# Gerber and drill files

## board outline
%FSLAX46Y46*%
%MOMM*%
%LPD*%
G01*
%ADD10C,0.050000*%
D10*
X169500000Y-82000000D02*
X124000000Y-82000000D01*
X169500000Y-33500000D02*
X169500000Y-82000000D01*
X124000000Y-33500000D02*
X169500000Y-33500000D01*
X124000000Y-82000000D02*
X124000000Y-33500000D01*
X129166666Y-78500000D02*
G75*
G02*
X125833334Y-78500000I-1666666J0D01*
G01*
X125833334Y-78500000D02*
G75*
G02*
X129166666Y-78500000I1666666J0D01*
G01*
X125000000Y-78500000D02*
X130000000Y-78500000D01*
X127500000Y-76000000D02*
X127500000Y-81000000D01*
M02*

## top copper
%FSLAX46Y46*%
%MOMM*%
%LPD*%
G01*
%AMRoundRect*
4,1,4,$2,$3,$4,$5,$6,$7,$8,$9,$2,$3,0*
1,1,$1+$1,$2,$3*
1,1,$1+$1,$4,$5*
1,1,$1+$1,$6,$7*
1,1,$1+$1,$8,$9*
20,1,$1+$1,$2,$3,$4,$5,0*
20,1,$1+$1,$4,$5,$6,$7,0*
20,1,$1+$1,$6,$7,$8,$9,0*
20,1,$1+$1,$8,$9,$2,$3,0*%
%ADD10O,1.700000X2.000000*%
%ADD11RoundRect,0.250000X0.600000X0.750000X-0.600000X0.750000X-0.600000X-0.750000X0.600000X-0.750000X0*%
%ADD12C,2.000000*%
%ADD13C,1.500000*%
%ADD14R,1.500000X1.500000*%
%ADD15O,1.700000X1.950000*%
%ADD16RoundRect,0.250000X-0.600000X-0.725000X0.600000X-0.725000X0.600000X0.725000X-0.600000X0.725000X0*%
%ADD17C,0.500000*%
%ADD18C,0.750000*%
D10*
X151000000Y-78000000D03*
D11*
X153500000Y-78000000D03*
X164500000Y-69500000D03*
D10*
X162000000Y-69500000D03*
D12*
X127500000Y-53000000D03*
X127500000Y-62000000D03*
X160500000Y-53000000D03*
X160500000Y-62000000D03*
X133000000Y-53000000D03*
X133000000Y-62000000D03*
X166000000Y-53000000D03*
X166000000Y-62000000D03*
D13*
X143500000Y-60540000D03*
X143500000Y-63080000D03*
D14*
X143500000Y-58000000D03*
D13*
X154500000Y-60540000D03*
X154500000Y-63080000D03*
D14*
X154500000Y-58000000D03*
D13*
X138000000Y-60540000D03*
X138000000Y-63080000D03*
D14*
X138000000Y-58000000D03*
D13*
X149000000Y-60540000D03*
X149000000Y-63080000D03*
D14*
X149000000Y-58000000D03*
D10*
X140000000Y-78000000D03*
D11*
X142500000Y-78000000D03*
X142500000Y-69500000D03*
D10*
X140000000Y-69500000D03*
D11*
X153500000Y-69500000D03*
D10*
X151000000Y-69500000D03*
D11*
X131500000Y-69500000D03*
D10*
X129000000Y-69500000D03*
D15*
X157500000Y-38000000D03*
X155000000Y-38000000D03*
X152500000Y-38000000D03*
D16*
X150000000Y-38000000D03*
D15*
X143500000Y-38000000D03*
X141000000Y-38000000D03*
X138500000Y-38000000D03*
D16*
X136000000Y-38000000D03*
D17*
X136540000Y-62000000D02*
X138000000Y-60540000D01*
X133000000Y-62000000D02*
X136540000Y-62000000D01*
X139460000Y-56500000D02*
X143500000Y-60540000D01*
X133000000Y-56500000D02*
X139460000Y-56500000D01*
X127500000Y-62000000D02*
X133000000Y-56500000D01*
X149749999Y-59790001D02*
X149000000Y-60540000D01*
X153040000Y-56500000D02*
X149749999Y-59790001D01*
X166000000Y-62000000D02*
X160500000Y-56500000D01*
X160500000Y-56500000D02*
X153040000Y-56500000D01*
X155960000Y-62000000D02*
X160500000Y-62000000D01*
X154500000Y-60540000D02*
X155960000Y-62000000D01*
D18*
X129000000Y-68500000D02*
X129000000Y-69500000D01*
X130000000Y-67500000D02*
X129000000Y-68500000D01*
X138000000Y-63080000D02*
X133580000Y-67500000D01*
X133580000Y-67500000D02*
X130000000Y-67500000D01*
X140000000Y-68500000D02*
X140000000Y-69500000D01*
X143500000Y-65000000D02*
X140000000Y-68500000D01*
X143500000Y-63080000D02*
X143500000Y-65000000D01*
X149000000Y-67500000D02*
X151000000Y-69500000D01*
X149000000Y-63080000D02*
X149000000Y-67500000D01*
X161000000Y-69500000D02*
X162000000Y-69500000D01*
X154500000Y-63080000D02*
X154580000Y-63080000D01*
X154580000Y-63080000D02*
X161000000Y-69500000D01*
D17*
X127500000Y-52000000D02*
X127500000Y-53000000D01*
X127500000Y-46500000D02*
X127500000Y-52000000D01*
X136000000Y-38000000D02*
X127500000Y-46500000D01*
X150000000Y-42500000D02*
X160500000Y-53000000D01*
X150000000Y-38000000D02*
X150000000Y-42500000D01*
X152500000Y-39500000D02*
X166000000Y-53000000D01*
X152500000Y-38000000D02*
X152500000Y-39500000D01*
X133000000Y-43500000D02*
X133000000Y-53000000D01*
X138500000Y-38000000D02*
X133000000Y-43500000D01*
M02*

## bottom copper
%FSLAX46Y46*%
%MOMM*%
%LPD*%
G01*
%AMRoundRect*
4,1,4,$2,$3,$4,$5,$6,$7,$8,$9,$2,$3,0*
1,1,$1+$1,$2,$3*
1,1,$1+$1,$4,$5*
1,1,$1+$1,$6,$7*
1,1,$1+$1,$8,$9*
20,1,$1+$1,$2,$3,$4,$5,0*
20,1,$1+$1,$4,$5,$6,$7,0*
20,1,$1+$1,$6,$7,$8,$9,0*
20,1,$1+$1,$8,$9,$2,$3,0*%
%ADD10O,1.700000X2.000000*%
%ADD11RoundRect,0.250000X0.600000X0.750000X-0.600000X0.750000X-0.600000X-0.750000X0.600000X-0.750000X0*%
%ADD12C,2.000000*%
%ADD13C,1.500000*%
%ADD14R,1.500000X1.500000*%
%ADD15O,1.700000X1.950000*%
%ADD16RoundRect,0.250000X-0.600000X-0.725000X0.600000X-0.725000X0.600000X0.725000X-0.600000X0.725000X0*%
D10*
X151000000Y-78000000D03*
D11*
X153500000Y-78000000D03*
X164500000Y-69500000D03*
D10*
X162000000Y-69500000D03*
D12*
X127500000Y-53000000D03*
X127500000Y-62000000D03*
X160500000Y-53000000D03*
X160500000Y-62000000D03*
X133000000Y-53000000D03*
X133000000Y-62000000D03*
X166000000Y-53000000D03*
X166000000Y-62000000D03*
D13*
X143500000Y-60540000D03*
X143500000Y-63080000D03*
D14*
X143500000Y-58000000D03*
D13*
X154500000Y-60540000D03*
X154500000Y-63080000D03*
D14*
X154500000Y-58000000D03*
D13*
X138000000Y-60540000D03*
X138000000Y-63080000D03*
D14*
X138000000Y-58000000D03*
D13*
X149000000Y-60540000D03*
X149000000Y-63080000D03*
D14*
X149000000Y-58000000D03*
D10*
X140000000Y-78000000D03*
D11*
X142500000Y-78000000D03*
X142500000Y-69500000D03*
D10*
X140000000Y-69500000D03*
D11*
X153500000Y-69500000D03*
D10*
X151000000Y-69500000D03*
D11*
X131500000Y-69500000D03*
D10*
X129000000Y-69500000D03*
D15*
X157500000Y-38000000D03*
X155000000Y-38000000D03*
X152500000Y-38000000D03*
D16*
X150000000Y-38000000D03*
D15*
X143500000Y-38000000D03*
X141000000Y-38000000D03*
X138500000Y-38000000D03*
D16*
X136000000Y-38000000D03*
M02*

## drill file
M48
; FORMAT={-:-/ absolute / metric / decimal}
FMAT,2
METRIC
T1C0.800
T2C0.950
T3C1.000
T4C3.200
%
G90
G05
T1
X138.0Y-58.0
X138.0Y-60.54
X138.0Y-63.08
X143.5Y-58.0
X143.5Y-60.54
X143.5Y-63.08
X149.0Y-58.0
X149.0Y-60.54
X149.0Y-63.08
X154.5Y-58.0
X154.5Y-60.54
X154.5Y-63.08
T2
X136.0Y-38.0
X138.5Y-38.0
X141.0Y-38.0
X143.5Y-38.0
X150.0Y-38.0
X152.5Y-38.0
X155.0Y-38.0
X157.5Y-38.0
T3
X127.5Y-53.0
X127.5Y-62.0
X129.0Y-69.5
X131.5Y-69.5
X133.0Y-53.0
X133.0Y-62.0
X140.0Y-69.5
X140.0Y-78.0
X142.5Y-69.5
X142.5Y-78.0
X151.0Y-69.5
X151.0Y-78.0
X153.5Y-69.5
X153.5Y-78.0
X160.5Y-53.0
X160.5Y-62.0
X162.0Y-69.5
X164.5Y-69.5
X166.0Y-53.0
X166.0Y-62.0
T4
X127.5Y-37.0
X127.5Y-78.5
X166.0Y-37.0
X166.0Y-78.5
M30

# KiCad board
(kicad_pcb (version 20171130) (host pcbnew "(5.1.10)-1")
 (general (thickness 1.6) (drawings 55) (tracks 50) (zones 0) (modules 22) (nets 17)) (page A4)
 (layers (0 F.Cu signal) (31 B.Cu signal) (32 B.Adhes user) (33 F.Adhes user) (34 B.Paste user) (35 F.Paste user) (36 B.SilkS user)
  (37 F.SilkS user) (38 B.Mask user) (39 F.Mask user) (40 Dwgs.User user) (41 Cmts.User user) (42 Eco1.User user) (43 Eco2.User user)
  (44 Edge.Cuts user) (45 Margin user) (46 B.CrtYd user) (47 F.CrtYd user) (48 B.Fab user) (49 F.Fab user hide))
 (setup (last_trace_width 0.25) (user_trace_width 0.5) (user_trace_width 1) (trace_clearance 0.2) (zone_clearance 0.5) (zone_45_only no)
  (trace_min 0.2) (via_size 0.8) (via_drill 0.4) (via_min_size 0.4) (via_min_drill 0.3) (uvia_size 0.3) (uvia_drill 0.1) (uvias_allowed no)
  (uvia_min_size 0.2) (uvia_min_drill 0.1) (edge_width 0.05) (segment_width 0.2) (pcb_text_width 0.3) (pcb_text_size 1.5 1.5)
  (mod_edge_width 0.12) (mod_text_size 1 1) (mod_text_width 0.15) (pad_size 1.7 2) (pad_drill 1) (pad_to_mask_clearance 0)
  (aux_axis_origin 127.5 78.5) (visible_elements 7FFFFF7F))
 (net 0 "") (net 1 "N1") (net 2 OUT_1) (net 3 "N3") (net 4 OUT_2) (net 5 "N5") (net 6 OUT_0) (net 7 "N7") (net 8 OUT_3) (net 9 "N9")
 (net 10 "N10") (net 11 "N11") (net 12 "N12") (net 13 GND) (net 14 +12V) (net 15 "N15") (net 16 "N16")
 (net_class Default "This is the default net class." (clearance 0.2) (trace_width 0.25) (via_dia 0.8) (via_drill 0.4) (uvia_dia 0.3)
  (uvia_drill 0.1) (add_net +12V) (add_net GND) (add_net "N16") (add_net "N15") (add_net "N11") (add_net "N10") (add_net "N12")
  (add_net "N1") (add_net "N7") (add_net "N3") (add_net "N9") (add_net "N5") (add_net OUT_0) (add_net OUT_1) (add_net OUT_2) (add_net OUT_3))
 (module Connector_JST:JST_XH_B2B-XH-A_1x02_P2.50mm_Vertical (layer F.Cu) (at 153.5 78 180)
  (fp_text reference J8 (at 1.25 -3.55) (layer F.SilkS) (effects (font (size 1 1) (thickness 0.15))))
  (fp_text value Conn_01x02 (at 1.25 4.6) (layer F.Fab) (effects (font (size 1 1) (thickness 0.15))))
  (pad 2 thru_hole oval (at 2.5 0 180) (size 1.7 2) (drill 1) (layers *.Cu *.Mask))
  (pad 1 thru_hole roundrect (at 0 0 180) (size 1.7 2) (drill 1) (layers *.Cu *.Mask) (roundrect_rratio 0.1470588235294118)))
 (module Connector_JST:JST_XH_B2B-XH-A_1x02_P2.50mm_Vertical (layer F.Cu) (at 164.5 69.5 180)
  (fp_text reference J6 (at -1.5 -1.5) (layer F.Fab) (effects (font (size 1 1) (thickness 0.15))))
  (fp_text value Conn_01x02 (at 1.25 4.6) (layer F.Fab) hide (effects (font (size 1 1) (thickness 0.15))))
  (pad 1 thru_hole roundrect (at 0 0 180) (size 1.7 2) (drill 1) (layers *.Cu *.Mask) (roundrect_rratio 0.1470588235294118))
  (pad 2 thru_hole oval (at 2.5 0 180) (size 1.7 2) (drill 1) (layers *.Cu *.Mask) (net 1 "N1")))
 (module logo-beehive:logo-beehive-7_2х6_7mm (layer F.Cu) (at 133 77 90)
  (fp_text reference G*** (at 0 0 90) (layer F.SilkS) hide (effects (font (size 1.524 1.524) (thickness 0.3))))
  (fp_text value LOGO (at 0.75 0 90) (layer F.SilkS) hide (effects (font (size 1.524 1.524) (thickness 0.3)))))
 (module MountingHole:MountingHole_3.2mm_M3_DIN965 (layer F.Cu) (at 166 37 270)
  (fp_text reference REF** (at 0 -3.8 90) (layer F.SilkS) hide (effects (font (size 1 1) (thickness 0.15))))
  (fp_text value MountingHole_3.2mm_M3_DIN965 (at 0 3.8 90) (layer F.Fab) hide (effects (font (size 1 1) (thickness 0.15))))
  (pad 1 np_thru_hole circle (at 0 0 270) (size 3.2 3.2) (drill 3.2) (layers *.Cu *.Mask)))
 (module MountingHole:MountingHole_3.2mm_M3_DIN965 (layer F.Cu) (at 166 78.5 180)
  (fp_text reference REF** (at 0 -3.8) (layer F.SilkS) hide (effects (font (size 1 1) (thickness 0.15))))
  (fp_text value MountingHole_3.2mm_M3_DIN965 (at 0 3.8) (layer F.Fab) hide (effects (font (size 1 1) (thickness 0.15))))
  (pad 1 np_thru_hole circle (at 0 0 180) (size 3.2 3.2) (drill 3.2) (layers *.Cu *.Mask)))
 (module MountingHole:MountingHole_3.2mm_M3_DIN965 (layer F.Cu) (at 127.5 78.5 90)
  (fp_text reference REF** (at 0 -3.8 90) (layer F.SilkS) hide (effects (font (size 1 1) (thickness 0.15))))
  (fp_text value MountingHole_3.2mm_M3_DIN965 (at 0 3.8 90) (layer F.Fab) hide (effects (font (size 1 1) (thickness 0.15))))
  (pad 1 np_thru_hole circle (at 0 0 90) (size 3.2 3.2) (drill 3.2) (layers *.Cu *.Mask)))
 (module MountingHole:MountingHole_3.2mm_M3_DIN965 (layer F.Cu) (at 127.5 37 90)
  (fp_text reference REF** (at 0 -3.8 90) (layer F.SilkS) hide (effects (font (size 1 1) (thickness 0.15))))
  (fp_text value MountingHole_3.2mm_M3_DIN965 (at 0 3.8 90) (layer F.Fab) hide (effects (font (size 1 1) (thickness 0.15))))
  (pad 1 np_thru_hole circle (at 0 0 90) (size 3.2 3.2) (drill 3.2) (layers *.Cu *.Mask)))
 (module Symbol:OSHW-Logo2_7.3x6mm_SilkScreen (layer F.Cu) (at 147 51)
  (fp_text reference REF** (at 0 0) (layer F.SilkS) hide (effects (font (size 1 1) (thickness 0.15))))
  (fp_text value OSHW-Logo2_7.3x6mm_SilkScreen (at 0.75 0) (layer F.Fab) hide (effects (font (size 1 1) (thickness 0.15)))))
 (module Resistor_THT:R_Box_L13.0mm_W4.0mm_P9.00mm (layer F.Cu) (at 127.5 53 270)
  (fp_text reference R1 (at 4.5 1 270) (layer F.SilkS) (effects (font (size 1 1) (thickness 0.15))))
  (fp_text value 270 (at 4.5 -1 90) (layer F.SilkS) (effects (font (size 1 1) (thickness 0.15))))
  (pad 1 thru_hole circle (at 0 0 270) (size 2 2) (drill 1) (layers *.Cu *.Mask) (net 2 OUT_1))
  (pad 2 thru_hole circle (at 9 0 270) (size 2 2) (drill 1) (layers *.Cu *.Mask) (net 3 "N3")))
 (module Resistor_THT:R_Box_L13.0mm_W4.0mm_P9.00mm (layer F.Cu) (at 160.5 53 270)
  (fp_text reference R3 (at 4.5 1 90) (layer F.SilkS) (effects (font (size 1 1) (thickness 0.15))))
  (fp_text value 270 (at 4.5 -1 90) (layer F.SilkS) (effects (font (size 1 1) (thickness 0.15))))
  (pad 1 thru_hole circle (at 0 0 270) (size 2 2) (drill 1) (layers *.Cu *.Mask) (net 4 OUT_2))
  (pad 2 thru_hole circle (at 9 0 270) (size 2 2) (drill 1) (layers *.Cu *.Mask) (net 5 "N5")))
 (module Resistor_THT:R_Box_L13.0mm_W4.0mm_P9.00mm (layer F.Cu) (at 133 53 270)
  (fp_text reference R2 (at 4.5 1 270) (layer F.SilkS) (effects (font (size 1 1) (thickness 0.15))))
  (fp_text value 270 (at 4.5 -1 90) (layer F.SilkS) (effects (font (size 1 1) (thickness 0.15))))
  (pad 1 thru_hole circle (at 0 0 270) (size 2 2) (drill 1) (layers *.Cu *.Mask) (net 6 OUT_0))
  (pad 2 thru_hole circle (at 9 0 270) (size 2 2) (drill 1) (layers *.Cu *.Mask) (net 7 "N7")))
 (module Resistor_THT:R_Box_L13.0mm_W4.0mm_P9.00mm (layer F.Cu) (at 166 53 270)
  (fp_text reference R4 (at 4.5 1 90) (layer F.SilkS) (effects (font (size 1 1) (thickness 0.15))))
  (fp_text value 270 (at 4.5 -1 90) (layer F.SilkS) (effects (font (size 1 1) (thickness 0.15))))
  (pad 1 thru_hole circle (at 0 0 270) (size 2 2) (drill 1) (layers *.Cu *.Mask) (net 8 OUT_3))
  (pad 2 thru_hole circle (at 9 0 270) (size 2 2) (drill 1) (layers *.Cu *.Mask) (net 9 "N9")))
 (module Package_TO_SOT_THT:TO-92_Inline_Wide (layer F.Cu) (at 143.5 58 270)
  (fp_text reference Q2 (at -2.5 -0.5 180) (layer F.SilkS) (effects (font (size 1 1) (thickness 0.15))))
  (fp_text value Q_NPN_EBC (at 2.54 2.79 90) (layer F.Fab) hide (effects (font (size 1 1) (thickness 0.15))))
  (pad 2 thru_hole circle (at 2.54 0) (size 1.5 1.5) (drill 0.8) (layers *.Cu *.Mask) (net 3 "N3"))
  (pad 3 thru_hole circle (at 5.08 0) (size 1.5 1.5) (drill 0.8) (layers *.Cu *.Mask) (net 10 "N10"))
  (pad 1 thru_hole rect (at 0 0) (size 1.5 1.5) (drill 0.8) (layers *.Cu *.Mask)))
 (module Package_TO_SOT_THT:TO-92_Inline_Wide (layer F.Cu) (at 154.5 58 270)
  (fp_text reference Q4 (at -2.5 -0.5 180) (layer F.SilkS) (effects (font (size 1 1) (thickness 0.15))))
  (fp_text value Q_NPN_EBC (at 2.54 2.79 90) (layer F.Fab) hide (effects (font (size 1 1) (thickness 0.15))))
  (pad 2 thru_hole circle (at 2.54 0) (size 1.5 1.5) (drill 0.8) (layers *.Cu *.Mask) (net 5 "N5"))
  (pad 3 thru_hole circle (at 5.08 0) (size 1.5 1.5) (drill 0.8) (layers *.Cu *.Mask) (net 1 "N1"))
  (pad 1 thru_hole rect (at 0 0) (size 1.5 1.5) (drill 0.8) (layers *.Cu *.Mask)))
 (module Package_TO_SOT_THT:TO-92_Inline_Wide (layer F.Cu) (at 138 58 270)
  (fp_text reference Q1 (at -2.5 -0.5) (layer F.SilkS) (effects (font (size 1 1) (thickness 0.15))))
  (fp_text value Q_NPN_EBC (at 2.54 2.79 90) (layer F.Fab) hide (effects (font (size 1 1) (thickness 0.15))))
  (pad 2 thru_hole circle (at 2.54 0) (size 1.5 1.5) (drill 0.8) (layers *.Cu *.Mask) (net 7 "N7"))
  (pad 3 thru_hole circle (at 5.08 0) (size 1.5 1.5) (drill 0.8) (layers *.Cu *.Mask) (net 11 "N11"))
  (pad 1 thru_hole rect (at 0 0) (size 1.5 1.5) (drill 0.8) (layers *.Cu *.Mask)))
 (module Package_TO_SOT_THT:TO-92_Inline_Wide (layer F.Cu) (at 149 58 270)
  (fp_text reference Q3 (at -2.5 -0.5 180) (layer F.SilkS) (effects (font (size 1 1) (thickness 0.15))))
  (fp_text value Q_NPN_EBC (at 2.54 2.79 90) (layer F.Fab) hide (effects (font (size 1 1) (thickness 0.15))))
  (pad 2 thru_hole circle (at 2.54 0) (size 1.5 1.5) (drill 0.8) (layers *.Cu *.Mask) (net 9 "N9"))
  (pad 3 thru_hole circle (at 5.08 0) (size 1.5 1.5) (drill 0.8) (layers *.Cu *.Mask) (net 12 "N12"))
  (pad 1 thru_hole rect (at 0 0) (size 1.5 1.5) (drill 0.8) (layers *.Cu *.Mask)))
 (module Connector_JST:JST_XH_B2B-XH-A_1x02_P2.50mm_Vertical (layer F.Cu) (at 142.5 78 180)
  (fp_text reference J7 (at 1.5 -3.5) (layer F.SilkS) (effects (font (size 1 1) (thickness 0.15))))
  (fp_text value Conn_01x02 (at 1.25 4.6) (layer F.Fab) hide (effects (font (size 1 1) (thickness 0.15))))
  (pad 2 thru_hole oval (at 2.5 0 180) (size 1.7 2) (drill 1) (layers *.Cu *.Mask))
  (pad 1 thru_hole roundrect (at 0 0 180) (size 1.7 2) (drill 1) (layers *.Cu *.Mask) (roundrect_rratio 0.1470588235294118)))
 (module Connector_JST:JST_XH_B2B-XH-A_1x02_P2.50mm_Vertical (layer F.Cu) (at 142.5 69.5 180)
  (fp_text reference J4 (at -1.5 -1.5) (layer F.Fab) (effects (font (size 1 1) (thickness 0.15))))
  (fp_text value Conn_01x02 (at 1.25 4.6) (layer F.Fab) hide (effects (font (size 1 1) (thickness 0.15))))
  (pad 1 thru_hole roundrect (at 0 0 180) (size 1.7 2) (drill 1) (layers *.Cu *.Mask) (roundrect_rratio 0.1470588235294118))
  (pad 2 thru_hole oval (at 2.5 0 180) (size 1.7 2) (drill 1) (layers *.Cu *.Mask) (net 10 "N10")))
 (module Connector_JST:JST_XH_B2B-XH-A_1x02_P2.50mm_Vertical (layer F.Cu) (at 153.5 69.5 180)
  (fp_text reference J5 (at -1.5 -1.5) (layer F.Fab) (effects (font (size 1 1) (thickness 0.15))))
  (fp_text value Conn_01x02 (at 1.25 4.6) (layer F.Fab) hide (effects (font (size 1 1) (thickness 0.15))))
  (pad 1 thru_hole roundrect (at 0 0 180) (size 1.7 2) (drill 1) (layers *.Cu *.Mask) (roundrect_rratio 0.1470588235294118))
  (pad 2 thru_hole oval (at 2.5 0 180) (size 1.7 2) (drill 1) (layers *.Cu *.Mask) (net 12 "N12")))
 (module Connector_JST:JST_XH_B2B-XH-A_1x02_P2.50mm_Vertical (layer F.Cu) (at 131.5 69.5 180)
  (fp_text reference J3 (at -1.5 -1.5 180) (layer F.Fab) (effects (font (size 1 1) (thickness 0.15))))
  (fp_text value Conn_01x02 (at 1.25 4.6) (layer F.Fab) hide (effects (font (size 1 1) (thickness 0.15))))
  (pad 1 thru_hole roundrect (at 0 0 180) (size 1.7 2) (drill 1) (layers *.Cu *.Mask) (roundrect_rratio 0.1470588235294118))
  (pad 2 thru_hole oval (at 2.5 0 180) (size 1.7 2) (drill 1) (layers *.Cu *.Mask) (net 11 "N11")))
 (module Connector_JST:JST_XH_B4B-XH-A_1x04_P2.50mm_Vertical (layer F.Cu) (at 150 38)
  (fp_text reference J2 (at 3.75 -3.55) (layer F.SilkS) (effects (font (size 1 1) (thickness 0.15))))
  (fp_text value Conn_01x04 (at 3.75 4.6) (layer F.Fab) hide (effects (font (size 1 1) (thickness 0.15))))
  (pad 4 thru_hole oval (at 7.5 0) (size 1.7 1.95) (drill 0.95) (layers *.Cu *.Mask))
  (pad 3 thru_hole oval (at 5 0) (size 1.7 1.95) (drill 0.95) (layers *.Cu *.Mask))
  (pad 2 thru_hole oval (at 2.5 0) (size 1.7 1.95) (drill 0.95) (layers *.Cu *.Mask) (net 8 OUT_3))
  (pad 1 thru_hole roundrect (at 0 0) (size 1.7 1.95) (drill 0.95) (layers *.Cu *.Mask) (roundrect_rratio 0.1470588235294118) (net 4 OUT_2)))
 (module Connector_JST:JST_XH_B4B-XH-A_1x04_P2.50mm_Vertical (layer F.Cu) (at 136 38)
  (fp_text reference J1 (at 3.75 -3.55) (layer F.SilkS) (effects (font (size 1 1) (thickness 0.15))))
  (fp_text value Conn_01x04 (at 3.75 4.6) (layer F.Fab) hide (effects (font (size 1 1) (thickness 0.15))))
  (pad 4 thru_hole oval (at 7.5 0) (size 1.7 1.95) (drill 0.95) (layers *.Cu *.Mask))
  (pad 3 thru_hole oval (at 5 0) (size 1.7 1.95) (drill 0.95) (layers *.Cu *.Mask))
  (pad 2 thru_hole oval (at 2.5 0) (size 1.7 1.95) (drill 0.95) (layers *.Cu *.Mask) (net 6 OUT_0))
  (pad 1 thru_hole roundrect (at 0 0) (size 1.7 1.95) (drill 0.95) (layers *.Cu *.Mask) (roundrect_rratio 0.1470588235294118) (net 2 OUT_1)))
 (gr_line (start 169.5 82) (end 124 82) (layer Edge.Cuts) (width 0.05))
 (gr_line (start 169.5 33.5) (end 169.5 82) (layer Edge.Cuts) (width 0.05))
 (gr_line (start 124 33.5) (end 169.5 33.5) (layer Edge.Cuts) (width 0.05))
 (gr_line (start 124 82) (end 124 33.5) (layer Edge.Cuts) (width 0.05))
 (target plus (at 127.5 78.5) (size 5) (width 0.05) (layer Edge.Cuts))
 (segment (start 136.54 62) (end 138 60.54) (width 0.5) (layer F.Cu) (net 7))
 (segment (start 133 62) (end 136.54 62) (width 0.5) (layer F.Cu) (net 7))
 (segment (start 139.46 56.5) (end 143.5 60.54) (width 0.5) (layer F.Cu) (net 3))
 (segment (start 133 56.5) (end 139.46 56.5) (width 0.5) (layer F.Cu) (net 3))
 (segment (start 127.5 62) (end 133 56.5) (width 0.5) (layer F.Cu) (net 3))
 (segment (start 149.749999 59.790001) (end 149 60.54) (width 0.5) (layer F.Cu) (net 9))
 (segment (start 153.04 56.5) (end 149.749999 59.790001) (width 0.5) (layer F.Cu) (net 9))
 (segment (start 166 62) (end 160.5 56.5) (width 0.5) (layer F.Cu) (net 9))
 (segment (start 160.5 56.5) (end 153.04 56.5) (width 0.5) (layer F.Cu) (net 9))
 (segment (start 155.96 62) (end 160.5 62) (width 0.5) (layer F.Cu) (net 5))
 (segment (start 154.5 60.54) (end 155.96 62) (width 0.5) (layer F.Cu) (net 5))
 (segment (start 129 68.5) (end 129 69.5) (width 0.75) (layer F.Cu) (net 11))
 (segment (start 130 67.5) (end 129 68.5) (width 0.75) (layer F.Cu) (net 11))
 (segment (start 138 63.08) (end 133.58 67.5) (width 0.75) (layer F.Cu) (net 11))
 (segment (start 133.58 67.5) (end 130 67.5) (width 0.75) (layer F.Cu) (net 11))
 (segment (start 140 68.5) (end 140 69.5) (width 0.75) (layer F.Cu) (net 10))
 (segment (start 143.5 65) (end 140 68.5) (width 0.75) (layer F.Cu) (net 10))
 (segment (start 143.5 63.08) (end 143.5 65) (width 0.75) (layer F.Cu) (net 10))
 (segment (start 149 67.5) (end 151 69.5) (width 0.75) (layer F.Cu) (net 12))
 (segment (start 149 63.08) (end 149 67.5) (width 0.75) (layer F.Cu) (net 12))
 (segment (start 161 69.5) (end 162 69.5) (width 0.75) (layer F.Cu) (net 1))
 (segment (start 154.5 63.08) (end 154.58 63.08) (width 0.75) (layer F.Cu) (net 1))
 (segment (start 154.58 63.08) (end 161 69.5) (width 0.75) (layer F.Cu) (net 1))
 (segment (start 127.5 52) (end 127.5 53) (width 0.5) (layer F.Cu) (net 2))
 (segment (start 127.5 46.5) (end 127.5 52) (width 0.5) (layer F.Cu) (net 2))
 (segment (start 136 38) (end 127.5 46.5) (width 0.5) (layer F.Cu) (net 2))
 (segment (start 150 42.5) (end 160.5 53) (width 0.5) (layer F.Cu) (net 4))
 (segment (start 150 38) (end 150 42.5) (width 0.5) (layer F.Cu) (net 4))
 (segment (start 152.5 39.5) (end 166 53) (width 0.5) (layer F.Cu) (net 8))
 (segment (start 152.5 38) (end 152.5 39.5) (width 0.5) (layer F.Cu) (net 8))
 (segment (start 133 43.5) (end 133 53) (width 0.5) (layer F.Cu) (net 6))
 (segment (start 138.5 38) (end 133 43.5) (width 0.5) (layer F.Cu) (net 6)))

